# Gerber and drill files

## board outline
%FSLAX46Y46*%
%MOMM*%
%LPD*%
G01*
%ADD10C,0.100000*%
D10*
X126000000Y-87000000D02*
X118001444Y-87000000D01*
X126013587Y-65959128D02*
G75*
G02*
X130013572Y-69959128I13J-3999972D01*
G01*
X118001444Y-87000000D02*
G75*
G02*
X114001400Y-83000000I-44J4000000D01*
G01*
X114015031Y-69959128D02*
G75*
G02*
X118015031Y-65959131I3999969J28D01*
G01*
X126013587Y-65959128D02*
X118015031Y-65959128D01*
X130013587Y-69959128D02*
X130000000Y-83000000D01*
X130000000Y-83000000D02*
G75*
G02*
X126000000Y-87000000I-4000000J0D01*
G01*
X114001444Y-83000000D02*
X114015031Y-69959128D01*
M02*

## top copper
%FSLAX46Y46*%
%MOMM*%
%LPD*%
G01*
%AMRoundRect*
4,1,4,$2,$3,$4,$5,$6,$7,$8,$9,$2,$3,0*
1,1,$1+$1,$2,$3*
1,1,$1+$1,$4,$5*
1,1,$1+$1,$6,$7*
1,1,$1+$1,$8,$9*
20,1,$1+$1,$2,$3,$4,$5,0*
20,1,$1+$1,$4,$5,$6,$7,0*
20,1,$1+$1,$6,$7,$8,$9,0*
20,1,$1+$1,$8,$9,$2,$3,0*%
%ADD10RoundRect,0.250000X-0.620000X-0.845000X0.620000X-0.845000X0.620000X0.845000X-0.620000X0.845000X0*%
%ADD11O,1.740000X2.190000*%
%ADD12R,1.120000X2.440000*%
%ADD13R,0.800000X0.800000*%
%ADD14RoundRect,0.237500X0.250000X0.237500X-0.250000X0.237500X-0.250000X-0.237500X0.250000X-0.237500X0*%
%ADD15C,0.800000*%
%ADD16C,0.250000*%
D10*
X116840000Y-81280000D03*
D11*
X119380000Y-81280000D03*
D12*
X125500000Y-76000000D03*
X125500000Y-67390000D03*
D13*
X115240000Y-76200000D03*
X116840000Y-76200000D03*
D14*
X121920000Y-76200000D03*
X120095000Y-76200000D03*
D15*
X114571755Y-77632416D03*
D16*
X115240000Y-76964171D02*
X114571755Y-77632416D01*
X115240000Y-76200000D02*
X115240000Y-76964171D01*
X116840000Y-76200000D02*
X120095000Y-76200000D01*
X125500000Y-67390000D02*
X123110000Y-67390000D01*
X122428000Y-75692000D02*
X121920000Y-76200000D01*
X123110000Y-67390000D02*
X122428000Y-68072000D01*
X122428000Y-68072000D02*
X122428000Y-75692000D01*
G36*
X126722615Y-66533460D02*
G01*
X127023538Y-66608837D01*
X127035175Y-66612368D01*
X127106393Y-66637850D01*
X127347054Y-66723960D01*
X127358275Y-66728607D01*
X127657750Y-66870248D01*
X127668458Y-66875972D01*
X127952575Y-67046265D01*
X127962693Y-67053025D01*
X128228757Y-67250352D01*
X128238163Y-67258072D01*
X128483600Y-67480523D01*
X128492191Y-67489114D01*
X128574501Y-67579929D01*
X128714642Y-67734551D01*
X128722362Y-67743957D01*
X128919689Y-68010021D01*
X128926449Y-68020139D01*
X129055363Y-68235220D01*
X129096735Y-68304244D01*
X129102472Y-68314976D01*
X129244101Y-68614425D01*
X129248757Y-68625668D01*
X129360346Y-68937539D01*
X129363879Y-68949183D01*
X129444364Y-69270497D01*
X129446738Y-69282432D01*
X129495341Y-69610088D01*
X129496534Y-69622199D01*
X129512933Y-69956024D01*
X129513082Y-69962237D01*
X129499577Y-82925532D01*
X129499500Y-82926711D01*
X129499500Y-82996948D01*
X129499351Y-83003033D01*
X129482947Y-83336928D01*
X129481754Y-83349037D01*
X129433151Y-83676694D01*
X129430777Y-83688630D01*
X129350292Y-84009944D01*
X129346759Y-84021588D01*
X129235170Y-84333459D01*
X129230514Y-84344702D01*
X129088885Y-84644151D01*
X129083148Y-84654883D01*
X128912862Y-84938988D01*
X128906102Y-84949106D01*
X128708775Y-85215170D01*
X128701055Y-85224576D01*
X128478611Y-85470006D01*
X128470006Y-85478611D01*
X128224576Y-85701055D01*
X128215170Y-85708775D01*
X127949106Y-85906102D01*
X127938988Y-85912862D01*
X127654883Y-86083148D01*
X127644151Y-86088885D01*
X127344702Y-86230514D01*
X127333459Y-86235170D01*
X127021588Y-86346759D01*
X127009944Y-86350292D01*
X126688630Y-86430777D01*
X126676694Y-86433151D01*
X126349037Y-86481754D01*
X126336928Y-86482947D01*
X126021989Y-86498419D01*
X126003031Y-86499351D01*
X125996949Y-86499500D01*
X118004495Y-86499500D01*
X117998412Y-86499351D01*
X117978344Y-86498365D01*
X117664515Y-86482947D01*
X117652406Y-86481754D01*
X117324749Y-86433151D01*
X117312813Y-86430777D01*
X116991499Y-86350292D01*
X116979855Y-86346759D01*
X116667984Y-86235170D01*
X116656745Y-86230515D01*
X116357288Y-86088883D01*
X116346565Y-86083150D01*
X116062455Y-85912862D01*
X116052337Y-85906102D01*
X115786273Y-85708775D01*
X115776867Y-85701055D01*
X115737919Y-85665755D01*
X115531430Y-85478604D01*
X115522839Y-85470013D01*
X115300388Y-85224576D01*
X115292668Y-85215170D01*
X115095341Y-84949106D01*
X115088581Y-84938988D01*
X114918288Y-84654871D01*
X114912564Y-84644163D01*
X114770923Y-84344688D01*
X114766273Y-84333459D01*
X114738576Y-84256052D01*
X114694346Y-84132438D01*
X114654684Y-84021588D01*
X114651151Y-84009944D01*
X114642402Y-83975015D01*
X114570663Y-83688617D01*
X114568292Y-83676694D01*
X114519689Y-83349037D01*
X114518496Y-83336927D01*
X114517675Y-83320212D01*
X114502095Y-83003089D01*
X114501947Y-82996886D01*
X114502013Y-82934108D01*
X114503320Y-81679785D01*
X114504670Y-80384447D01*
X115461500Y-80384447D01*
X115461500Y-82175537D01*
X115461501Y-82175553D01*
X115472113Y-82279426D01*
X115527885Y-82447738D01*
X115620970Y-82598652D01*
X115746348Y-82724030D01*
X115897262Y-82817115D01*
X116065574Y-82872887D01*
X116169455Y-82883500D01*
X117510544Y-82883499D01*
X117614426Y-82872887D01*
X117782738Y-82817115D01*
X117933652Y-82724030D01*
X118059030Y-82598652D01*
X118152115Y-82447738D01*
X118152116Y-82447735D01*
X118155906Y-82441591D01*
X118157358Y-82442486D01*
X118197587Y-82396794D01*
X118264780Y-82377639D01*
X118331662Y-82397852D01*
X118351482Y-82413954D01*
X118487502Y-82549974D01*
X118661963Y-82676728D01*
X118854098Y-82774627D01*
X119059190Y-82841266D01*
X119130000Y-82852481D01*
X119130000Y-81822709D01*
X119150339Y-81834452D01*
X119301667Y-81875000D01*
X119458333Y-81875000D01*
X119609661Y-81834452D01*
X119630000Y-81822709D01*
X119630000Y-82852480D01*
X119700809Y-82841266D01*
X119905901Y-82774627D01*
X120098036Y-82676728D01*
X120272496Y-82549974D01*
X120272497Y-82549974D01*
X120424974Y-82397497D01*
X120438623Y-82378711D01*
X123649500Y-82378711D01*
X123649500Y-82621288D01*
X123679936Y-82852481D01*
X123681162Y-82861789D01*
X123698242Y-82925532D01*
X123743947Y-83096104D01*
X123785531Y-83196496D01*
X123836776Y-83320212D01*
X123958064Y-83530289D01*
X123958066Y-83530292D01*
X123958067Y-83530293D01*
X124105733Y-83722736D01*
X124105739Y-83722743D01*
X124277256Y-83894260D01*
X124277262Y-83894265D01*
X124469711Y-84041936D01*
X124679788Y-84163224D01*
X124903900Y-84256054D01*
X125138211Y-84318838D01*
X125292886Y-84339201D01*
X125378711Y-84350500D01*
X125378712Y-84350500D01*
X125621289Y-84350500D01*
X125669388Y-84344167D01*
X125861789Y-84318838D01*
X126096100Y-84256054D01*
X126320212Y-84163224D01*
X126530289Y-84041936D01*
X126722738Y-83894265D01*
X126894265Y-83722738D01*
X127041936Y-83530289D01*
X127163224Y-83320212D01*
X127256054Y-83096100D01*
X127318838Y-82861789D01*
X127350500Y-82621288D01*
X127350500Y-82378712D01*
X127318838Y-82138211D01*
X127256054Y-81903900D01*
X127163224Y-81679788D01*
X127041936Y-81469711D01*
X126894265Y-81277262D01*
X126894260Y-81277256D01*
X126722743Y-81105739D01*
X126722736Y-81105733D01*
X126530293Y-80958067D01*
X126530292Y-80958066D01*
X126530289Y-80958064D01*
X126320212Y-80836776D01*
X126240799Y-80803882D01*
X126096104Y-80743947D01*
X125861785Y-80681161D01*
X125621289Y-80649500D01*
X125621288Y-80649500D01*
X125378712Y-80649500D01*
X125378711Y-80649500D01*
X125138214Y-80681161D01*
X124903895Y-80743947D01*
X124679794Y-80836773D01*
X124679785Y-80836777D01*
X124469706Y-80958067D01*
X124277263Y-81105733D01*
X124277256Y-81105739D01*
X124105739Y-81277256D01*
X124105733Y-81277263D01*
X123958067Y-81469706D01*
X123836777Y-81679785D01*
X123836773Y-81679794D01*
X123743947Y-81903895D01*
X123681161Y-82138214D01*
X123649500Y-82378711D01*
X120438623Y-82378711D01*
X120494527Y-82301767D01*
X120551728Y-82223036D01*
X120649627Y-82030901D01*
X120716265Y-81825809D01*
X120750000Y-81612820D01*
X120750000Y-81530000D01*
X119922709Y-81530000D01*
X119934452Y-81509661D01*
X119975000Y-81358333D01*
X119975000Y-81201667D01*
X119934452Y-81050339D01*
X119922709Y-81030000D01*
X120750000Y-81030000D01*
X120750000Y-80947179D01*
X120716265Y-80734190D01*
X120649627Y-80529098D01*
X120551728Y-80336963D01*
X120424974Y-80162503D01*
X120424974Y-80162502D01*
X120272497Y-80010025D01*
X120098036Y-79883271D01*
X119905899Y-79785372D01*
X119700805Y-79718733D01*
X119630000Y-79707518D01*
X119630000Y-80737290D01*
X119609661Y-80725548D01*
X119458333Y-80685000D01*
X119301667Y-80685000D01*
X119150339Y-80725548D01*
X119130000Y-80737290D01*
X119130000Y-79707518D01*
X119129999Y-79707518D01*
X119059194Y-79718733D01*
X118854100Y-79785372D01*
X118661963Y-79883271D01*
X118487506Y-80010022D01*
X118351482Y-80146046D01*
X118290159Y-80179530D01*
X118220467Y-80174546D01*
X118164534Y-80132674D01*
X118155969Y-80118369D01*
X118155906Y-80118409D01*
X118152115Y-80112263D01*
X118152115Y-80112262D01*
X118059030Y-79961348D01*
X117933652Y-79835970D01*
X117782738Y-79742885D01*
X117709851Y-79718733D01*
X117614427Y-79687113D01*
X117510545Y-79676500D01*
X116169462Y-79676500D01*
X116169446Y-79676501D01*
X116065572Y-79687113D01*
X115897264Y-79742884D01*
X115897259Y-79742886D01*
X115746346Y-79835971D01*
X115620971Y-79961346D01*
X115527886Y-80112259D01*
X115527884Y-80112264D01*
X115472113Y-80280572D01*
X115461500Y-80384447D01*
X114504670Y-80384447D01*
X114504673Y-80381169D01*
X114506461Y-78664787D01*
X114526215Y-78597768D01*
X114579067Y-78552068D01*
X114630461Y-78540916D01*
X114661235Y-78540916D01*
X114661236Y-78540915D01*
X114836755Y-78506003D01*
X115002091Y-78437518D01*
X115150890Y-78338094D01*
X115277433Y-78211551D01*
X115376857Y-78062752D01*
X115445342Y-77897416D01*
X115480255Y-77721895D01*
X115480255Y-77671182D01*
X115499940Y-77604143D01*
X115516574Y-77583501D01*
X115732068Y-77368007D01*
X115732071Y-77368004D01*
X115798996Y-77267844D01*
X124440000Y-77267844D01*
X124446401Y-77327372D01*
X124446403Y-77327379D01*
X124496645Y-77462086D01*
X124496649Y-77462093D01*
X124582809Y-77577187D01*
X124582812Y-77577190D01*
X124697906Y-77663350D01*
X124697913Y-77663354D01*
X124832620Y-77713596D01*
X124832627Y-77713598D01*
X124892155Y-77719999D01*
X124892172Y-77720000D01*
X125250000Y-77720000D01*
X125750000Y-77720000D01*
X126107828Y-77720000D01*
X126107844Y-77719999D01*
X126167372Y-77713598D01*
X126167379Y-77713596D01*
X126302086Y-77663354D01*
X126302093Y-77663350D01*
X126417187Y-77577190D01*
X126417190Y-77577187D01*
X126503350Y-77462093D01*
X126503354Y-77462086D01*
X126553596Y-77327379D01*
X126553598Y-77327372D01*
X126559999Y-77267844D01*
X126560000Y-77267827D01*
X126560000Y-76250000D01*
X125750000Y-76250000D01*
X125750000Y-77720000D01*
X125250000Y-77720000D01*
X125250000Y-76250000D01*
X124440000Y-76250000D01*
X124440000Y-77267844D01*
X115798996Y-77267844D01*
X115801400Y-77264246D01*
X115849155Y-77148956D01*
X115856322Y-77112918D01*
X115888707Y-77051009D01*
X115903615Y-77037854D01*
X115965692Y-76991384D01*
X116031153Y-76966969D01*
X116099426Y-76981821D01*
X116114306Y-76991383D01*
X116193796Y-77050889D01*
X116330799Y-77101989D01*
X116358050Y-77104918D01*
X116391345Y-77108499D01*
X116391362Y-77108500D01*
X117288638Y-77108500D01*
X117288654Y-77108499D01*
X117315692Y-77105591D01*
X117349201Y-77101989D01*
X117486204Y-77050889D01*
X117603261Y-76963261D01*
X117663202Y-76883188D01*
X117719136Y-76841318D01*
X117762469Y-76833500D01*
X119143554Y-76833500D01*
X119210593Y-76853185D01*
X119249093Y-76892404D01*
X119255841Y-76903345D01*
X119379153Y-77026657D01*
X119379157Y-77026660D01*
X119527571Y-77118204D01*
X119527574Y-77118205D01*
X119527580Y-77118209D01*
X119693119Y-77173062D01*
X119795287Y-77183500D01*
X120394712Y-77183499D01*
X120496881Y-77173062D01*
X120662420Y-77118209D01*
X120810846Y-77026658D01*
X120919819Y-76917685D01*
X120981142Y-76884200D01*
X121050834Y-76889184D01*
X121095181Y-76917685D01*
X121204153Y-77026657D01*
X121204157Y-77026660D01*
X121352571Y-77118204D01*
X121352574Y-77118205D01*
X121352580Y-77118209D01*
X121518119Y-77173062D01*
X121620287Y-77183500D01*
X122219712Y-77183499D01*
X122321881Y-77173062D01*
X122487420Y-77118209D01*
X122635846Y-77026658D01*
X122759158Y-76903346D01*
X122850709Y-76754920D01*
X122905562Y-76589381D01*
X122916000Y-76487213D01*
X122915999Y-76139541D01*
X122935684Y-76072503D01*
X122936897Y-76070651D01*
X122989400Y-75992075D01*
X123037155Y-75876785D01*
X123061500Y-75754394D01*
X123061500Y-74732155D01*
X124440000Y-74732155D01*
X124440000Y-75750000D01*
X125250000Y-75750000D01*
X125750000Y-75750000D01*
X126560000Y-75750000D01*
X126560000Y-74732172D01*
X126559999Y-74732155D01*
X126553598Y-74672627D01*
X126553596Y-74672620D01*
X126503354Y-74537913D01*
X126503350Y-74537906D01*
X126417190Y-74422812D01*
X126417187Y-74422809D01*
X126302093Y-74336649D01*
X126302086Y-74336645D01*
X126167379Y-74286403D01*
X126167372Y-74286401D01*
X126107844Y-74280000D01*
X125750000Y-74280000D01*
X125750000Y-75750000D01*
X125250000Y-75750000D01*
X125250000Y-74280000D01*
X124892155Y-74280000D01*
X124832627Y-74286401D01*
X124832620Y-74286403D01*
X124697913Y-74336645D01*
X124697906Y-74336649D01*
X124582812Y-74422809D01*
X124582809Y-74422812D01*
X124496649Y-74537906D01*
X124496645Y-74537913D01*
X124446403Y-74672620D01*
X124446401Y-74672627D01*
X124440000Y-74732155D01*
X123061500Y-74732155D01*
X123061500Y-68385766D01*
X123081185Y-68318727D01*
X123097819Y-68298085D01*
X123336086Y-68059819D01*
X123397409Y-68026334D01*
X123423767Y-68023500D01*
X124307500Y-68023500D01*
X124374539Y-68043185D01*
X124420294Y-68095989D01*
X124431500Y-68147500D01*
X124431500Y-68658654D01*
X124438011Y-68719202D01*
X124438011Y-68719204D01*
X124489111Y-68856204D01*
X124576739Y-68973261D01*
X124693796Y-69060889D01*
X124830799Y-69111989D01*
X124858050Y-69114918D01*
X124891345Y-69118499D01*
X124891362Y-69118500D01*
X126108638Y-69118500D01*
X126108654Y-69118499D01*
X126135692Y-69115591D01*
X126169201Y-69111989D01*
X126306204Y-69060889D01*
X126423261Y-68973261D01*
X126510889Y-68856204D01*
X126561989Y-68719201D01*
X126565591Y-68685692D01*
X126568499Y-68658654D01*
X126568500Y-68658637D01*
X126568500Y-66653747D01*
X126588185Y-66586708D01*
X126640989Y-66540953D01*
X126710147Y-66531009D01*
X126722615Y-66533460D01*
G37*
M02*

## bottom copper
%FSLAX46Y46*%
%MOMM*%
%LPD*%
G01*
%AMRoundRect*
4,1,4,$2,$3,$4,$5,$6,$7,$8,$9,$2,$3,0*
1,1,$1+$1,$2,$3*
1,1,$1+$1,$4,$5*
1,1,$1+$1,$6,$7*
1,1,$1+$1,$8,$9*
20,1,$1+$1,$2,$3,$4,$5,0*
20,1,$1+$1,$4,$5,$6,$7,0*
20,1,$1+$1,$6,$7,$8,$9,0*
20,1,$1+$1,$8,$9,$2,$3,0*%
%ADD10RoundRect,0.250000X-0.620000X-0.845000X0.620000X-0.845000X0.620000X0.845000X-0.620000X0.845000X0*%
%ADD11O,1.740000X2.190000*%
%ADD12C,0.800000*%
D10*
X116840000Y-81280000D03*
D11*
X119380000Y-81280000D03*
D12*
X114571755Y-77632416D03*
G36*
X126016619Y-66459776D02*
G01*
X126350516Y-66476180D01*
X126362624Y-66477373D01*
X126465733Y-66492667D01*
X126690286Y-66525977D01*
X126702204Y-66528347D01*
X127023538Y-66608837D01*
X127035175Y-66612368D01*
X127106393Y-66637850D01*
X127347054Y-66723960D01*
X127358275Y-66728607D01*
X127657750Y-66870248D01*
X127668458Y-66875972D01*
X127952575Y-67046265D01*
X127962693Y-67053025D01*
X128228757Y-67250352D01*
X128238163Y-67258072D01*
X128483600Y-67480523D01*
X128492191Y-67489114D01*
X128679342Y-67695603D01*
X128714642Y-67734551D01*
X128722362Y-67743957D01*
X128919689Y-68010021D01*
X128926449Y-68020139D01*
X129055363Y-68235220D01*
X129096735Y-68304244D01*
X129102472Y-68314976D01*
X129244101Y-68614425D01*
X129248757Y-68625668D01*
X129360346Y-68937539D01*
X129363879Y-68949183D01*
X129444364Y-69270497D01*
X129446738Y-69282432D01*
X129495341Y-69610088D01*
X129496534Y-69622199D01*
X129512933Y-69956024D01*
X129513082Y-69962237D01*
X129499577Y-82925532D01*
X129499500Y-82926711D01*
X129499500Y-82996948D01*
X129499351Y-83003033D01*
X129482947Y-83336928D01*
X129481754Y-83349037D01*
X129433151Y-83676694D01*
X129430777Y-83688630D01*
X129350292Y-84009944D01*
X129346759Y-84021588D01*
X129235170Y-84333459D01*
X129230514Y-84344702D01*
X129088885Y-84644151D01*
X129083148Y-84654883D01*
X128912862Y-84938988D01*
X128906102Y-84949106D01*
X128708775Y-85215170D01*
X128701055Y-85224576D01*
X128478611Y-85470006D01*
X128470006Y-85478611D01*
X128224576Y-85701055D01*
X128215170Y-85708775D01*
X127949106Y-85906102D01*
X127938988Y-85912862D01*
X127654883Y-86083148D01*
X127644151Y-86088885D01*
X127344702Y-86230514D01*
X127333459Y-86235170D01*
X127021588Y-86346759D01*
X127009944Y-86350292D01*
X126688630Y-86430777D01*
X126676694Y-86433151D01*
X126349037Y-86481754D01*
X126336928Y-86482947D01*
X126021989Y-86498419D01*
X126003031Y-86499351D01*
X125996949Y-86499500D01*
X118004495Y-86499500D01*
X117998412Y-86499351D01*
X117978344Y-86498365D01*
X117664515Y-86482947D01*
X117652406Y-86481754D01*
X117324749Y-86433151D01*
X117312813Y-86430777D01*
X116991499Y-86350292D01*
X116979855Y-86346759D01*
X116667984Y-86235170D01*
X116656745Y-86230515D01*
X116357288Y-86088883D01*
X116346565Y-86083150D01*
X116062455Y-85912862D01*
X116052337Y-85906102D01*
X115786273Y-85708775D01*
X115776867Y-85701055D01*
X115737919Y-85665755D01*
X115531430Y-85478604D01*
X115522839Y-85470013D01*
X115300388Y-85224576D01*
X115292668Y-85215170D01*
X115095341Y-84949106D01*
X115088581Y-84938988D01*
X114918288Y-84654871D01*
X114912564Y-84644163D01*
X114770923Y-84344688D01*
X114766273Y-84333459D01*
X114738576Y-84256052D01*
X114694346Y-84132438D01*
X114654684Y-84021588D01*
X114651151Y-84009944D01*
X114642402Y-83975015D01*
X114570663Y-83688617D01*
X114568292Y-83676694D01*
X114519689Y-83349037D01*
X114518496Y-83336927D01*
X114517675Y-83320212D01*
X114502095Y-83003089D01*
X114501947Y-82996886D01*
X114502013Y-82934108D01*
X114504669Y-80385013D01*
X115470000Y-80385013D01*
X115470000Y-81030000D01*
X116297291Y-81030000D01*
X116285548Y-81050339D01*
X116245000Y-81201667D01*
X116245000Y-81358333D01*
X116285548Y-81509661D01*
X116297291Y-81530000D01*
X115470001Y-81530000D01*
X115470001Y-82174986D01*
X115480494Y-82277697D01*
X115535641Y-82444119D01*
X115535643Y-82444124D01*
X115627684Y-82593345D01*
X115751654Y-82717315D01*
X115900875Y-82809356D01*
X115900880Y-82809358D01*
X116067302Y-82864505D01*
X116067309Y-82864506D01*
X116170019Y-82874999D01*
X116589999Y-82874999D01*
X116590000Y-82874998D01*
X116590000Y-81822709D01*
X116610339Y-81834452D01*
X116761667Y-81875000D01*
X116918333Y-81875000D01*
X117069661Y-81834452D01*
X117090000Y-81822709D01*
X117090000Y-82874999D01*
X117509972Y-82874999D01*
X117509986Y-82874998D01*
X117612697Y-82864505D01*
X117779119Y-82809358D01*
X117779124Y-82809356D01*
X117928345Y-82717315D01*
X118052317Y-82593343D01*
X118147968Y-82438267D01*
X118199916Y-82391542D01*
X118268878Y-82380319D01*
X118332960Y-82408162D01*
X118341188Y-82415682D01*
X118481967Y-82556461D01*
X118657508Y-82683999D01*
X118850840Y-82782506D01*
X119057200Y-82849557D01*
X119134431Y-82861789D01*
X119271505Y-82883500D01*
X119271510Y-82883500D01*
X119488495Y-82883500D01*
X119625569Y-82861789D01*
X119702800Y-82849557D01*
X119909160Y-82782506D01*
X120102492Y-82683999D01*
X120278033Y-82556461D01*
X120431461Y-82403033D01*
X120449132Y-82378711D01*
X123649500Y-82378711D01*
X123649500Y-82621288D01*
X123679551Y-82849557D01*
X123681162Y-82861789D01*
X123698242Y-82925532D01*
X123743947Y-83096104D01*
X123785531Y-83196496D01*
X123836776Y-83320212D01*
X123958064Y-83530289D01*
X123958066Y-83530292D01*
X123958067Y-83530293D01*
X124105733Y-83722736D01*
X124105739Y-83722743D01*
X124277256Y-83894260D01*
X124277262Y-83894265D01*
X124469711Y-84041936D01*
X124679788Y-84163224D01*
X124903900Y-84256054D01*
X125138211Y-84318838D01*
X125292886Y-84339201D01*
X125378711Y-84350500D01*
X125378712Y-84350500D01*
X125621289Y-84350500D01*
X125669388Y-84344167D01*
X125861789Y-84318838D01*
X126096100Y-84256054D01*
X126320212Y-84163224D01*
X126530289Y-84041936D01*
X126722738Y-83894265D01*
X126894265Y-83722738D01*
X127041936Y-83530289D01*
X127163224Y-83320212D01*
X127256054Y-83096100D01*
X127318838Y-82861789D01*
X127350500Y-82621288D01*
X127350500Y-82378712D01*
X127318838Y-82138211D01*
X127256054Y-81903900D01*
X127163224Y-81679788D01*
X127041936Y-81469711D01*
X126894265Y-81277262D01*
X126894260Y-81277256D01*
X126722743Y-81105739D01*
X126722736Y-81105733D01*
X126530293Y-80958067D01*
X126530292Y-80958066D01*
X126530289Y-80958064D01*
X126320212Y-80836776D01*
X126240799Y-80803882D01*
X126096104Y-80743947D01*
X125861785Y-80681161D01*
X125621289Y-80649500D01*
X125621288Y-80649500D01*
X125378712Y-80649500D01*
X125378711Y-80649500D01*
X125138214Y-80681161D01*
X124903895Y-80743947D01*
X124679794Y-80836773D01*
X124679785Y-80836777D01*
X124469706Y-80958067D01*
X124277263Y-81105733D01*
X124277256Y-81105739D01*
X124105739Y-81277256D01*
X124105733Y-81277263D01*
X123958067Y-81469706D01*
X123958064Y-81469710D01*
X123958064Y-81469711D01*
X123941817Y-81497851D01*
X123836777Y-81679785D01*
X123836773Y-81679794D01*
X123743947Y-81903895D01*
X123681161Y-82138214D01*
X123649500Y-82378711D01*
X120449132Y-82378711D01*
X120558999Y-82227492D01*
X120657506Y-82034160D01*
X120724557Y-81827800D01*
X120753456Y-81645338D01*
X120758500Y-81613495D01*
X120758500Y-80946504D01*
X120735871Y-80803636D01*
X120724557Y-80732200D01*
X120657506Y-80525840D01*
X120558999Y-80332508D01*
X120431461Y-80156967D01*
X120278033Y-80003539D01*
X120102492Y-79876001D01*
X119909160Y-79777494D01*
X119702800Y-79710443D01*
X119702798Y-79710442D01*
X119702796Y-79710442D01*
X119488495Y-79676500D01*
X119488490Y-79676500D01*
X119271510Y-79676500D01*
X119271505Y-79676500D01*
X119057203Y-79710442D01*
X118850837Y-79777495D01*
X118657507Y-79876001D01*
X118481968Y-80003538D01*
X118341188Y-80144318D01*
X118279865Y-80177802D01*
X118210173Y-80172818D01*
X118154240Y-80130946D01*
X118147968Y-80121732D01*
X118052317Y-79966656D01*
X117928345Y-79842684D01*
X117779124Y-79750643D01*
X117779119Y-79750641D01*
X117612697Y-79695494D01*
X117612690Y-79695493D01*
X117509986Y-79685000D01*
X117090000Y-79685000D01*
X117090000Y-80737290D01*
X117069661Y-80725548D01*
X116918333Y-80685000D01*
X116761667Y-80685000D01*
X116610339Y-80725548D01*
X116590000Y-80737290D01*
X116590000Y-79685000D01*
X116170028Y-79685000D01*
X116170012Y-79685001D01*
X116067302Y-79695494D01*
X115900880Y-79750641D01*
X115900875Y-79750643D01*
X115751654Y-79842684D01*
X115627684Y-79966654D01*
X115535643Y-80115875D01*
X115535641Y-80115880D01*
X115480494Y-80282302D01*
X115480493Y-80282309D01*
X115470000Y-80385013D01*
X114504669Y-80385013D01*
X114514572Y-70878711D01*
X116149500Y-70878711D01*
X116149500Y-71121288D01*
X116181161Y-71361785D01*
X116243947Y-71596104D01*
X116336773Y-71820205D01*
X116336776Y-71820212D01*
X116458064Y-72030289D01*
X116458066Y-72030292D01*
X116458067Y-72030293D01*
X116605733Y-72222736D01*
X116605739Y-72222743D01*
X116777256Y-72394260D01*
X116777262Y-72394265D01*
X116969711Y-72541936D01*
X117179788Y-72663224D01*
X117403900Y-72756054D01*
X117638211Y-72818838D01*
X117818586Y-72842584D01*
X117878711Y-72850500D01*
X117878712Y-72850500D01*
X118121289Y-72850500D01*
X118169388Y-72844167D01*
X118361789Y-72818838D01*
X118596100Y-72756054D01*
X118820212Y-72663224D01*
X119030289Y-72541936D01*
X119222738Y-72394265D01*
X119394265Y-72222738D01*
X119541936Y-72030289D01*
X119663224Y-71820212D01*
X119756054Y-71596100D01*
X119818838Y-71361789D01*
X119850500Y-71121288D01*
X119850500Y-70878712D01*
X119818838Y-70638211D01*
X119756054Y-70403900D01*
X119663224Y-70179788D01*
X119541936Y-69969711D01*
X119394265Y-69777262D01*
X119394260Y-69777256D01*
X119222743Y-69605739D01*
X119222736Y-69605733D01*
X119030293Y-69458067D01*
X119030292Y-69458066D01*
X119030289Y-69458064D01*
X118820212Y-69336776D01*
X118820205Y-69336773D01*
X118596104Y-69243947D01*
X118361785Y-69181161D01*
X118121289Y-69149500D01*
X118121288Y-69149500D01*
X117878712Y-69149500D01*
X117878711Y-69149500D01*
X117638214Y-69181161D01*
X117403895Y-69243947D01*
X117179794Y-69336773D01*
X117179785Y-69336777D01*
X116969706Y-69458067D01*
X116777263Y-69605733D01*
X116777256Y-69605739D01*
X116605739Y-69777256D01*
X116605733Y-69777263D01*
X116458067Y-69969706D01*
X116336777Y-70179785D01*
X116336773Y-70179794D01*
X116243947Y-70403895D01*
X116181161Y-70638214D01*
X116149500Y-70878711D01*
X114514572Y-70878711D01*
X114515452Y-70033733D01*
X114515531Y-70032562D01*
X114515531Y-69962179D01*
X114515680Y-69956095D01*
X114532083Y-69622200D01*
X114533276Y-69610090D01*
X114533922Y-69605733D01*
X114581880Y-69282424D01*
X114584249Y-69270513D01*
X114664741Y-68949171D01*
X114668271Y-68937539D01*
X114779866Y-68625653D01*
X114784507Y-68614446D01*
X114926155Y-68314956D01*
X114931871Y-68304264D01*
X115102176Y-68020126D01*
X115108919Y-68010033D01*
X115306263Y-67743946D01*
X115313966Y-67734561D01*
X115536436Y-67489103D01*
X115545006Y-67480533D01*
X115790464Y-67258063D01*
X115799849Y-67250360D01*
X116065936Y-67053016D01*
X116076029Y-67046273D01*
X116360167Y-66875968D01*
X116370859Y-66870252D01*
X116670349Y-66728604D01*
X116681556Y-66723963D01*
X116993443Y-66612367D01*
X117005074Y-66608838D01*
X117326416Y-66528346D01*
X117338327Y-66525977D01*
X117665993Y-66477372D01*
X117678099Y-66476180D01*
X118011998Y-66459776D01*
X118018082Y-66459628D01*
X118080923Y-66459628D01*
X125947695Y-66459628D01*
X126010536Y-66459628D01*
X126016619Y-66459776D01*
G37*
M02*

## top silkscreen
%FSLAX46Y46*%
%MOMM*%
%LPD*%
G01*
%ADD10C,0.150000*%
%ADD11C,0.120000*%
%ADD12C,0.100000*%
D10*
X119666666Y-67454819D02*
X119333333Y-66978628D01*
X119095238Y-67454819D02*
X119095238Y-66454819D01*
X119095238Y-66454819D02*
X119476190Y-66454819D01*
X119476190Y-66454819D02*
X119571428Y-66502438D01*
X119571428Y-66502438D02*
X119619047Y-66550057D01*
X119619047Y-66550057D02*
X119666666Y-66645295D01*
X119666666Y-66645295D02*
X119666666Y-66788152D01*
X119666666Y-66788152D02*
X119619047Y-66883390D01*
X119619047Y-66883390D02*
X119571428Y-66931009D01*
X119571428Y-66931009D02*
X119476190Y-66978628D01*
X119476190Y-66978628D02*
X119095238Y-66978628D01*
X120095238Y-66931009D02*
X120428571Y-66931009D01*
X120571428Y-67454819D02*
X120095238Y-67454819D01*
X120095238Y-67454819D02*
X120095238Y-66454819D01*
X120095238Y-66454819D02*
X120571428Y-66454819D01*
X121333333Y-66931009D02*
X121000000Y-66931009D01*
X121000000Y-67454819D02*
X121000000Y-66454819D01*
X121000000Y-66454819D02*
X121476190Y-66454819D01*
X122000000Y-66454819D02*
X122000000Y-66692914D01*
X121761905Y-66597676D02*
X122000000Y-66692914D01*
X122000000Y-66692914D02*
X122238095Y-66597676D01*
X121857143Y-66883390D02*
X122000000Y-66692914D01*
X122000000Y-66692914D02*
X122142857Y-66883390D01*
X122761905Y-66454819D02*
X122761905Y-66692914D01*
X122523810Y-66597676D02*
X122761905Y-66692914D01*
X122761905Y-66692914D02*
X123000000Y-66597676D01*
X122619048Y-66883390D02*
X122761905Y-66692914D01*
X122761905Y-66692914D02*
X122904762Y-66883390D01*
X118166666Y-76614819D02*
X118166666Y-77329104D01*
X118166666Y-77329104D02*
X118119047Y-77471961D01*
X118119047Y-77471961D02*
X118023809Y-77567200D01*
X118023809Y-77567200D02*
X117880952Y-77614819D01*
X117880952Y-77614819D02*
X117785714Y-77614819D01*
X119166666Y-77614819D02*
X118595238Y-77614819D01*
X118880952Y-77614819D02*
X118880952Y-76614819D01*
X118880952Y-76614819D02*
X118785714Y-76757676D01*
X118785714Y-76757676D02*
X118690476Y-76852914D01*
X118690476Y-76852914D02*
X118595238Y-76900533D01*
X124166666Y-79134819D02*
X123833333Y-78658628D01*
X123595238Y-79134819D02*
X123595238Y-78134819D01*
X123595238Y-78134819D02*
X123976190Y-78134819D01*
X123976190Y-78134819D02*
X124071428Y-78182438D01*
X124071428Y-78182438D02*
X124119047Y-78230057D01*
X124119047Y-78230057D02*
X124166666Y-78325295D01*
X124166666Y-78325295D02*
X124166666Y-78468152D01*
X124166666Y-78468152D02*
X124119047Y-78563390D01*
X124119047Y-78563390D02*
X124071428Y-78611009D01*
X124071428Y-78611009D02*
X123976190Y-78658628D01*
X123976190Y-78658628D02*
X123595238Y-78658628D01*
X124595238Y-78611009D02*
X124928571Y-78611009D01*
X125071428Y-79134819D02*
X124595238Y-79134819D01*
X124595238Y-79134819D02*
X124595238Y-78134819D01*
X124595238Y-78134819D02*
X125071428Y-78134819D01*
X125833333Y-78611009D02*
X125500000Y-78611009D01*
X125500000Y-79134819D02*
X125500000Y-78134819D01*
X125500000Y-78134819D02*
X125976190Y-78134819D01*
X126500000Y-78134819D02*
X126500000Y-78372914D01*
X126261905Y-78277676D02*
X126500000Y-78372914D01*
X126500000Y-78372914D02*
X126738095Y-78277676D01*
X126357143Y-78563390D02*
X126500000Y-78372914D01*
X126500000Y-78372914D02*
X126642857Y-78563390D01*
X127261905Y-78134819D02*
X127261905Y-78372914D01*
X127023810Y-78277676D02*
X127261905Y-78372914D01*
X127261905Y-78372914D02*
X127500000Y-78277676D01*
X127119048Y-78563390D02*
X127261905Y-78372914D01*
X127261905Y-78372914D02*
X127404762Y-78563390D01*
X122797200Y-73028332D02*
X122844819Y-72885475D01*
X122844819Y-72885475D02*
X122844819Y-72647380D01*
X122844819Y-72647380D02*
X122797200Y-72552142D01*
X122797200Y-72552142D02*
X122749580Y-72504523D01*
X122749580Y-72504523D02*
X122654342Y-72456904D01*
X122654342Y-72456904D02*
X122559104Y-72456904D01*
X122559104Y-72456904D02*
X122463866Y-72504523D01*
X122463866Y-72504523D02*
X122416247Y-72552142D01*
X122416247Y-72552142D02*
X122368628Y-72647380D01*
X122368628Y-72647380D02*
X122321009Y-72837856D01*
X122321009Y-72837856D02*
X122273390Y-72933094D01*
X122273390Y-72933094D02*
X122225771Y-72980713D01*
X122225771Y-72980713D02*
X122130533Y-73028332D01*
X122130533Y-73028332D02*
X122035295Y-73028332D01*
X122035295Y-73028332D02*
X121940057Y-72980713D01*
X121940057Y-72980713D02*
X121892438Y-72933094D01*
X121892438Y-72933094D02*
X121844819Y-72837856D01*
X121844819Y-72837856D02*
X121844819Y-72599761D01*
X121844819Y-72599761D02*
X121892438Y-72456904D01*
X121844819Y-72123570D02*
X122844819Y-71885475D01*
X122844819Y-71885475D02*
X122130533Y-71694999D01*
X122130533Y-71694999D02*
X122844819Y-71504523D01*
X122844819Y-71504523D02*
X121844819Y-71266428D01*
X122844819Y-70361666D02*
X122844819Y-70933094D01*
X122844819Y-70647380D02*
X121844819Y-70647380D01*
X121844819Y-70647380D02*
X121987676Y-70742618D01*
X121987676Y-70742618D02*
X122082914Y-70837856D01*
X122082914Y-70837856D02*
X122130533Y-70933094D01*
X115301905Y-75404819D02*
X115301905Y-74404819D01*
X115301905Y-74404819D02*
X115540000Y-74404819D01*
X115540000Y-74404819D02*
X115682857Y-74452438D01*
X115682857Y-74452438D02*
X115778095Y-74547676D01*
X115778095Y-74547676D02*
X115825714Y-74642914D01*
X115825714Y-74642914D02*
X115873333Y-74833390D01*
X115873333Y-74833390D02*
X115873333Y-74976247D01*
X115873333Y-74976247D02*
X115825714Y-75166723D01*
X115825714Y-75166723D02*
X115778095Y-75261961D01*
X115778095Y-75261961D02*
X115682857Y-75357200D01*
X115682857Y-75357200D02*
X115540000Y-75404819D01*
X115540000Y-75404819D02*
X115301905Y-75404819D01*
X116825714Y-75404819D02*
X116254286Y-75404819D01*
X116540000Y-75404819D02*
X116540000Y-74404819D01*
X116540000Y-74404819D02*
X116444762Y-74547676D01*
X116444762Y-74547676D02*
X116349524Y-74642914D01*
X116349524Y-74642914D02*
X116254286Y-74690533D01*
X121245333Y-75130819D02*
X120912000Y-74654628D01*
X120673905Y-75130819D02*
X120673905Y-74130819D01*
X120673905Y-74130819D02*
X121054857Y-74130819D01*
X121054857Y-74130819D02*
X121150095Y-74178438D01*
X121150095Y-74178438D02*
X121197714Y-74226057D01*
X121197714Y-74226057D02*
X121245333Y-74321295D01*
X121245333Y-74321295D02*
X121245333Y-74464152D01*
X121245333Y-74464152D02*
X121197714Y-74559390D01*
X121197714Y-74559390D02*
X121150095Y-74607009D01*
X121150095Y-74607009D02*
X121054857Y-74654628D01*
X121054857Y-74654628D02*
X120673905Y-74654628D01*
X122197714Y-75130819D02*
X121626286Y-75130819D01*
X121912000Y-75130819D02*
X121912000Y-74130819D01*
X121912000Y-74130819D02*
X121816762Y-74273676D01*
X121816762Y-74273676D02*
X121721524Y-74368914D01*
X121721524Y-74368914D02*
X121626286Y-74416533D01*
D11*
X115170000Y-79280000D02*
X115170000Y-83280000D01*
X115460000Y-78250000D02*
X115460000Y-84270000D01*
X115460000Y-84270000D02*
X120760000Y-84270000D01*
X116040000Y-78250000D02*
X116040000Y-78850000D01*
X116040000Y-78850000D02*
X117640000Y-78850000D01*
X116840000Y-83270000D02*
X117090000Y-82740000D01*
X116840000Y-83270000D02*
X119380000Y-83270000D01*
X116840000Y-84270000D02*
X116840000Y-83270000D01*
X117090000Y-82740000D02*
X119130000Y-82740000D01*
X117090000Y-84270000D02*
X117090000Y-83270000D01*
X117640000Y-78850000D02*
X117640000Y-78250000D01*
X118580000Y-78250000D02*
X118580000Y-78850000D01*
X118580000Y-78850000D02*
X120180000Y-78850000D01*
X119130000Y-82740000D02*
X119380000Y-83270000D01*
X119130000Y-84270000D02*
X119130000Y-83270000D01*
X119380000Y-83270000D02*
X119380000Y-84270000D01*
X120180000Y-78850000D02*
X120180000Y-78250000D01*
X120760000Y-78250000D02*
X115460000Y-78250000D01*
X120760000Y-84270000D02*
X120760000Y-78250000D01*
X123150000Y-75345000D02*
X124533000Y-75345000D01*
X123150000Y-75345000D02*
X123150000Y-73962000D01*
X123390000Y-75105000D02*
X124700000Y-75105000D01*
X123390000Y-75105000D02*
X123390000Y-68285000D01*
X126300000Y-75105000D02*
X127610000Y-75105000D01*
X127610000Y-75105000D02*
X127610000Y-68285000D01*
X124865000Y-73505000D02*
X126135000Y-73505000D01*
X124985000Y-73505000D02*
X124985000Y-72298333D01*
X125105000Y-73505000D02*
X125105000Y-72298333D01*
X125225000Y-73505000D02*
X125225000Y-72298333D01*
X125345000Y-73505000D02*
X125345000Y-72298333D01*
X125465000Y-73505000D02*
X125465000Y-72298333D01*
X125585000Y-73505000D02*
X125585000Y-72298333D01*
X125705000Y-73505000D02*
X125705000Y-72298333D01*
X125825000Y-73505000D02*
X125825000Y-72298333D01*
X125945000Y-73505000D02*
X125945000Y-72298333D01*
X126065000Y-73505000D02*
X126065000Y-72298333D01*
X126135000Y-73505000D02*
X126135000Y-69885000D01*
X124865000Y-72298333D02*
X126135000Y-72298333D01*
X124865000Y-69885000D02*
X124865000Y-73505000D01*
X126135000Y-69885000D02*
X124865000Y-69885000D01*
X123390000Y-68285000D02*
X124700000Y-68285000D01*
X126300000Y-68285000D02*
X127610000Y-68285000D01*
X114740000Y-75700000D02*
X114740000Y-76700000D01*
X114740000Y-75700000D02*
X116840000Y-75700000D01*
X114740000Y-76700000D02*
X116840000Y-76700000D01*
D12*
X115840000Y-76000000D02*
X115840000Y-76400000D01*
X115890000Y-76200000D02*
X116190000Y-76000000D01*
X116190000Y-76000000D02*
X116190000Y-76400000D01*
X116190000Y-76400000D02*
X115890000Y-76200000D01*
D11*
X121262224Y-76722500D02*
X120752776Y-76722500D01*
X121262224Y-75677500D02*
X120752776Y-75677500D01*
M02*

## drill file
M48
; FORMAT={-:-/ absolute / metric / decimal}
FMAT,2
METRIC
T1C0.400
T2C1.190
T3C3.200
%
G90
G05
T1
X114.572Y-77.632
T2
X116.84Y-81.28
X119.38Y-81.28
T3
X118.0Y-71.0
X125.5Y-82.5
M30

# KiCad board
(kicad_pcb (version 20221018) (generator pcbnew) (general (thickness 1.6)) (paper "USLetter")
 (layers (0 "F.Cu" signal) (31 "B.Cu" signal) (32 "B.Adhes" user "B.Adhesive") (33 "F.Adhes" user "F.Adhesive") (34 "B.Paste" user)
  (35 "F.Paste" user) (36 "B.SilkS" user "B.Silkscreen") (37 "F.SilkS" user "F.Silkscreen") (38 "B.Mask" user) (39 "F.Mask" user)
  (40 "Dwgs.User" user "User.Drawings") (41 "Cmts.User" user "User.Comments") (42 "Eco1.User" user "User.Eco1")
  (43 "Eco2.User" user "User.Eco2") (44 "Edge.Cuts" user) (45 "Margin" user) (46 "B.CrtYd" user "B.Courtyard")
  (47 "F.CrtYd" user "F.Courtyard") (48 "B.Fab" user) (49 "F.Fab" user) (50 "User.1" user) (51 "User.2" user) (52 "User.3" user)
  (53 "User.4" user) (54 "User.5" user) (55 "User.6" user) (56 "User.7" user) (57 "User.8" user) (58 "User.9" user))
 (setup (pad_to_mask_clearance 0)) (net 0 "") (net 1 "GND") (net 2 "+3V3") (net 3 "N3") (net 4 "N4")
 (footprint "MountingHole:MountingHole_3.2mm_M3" (layer "F.Cu") (at 118 71)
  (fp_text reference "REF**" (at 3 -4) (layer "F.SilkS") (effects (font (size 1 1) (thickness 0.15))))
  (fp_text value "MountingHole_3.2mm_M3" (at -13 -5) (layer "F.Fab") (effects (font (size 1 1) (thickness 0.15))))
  (pad "" np_thru_hole circle (at 0 0) (size 3.2 3.2) (drill 3.2) (layers "*.Cu" "*.Mask")))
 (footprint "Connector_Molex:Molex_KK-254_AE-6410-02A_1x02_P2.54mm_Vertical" (layer "F.Cu") (at 116.84 81.28)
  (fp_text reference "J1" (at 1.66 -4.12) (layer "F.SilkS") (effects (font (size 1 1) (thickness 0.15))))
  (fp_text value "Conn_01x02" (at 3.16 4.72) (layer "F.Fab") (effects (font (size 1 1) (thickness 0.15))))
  (fp_line (start -1.67 -2) (end -1.67 2) (stroke (width 0.12) (type solid)) (layer "F.SilkS"))
  (fp_line (start -1.38 -3.03) (end -1.38 2.99) (stroke (width 0.12) (type solid)) (layer "F.SilkS"))
  (fp_line (start -1.38 2.99) (end 3.92 2.99) (stroke (width 0.12) (type solid)) (layer "F.SilkS"))
  (fp_line (start -0.8 -3.03) (end -0.8 -2.43) (stroke (width 0.12) (type solid)) (layer "F.SilkS"))
  (fp_line (start -0.8 -2.43) (end 0.8 -2.43) (stroke (width 0.12) (type solid)) (layer "F.SilkS"))
  (fp_line (start 0 1.99) (end 0.25 1.46) (stroke (width 0.12) (type solid)) (layer "F.SilkS"))
  (fp_line (start 0 1.99) (end 2.54 1.99) (stroke (width 0.12) (type solid)) (layer "F.SilkS"))
  (fp_line (start 0 2.99) (end 0 1.99) (stroke (width 0.12) (type solid)) (layer "F.SilkS"))
  (fp_line (start 0.25 1.46) (end 2.29 1.46) (stroke (width 0.12) (type solid)) (layer "F.SilkS"))
  (fp_line (start 0.25 2.99) (end 0.25 1.99) (stroke (width 0.12) (type solid)) (layer "F.SilkS"))
  (fp_line (start 0.8 -2.43) (end 0.8 -3.03) (stroke (width 0.12) (type solid)) (layer "F.SilkS"))
  (fp_line (start 1.74 -3.03) (end 1.74 -2.43) (stroke (width 0.12) (type solid)) (layer "F.SilkS"))
  (fp_line (start 1.74 -2.43) (end 3.34 -2.43) (stroke (width 0.12) (type solid)) (layer "F.SilkS"))
  (fp_line (start 2.29 1.46) (end 2.54 1.99) (stroke (width 0.12) (type solid)) (layer "F.SilkS"))
  (fp_line (start 2.29 2.99) (end 2.29 1.99) (stroke (width 0.12) (type solid)) (layer "F.SilkS"))
  (fp_line (start 2.54 1.99) (end 2.54 2.99) (stroke (width 0.12) (type solid)) (layer "F.SilkS"))
  (fp_line (start 3.34 -2.43) (end 3.34 -3.03) (stroke (width 0.12) (type solid)) (layer "F.SilkS"))
  (fp_line (start 3.92 -3.03) (end -1.38 -3.03) (stroke (width 0.12) (type solid)) (layer "F.SilkS"))
  (fp_line (start 3.92 2.99) (end 3.92 -3.03) (stroke (width 0.12) (type solid)) (layer "F.SilkS"))
  (pad "1" thru_hole roundrect (at 0 0) (size 1.74 2.19) (drill 1.19) (layers "*.Cu" "*.Mask") (roundrect_rratio 0.143678) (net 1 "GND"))
  (pad "2" thru_hole oval (at 2.54 0) (size 1.74 2.19) (drill 1.19) (layers "*.Cu" "*.Mask") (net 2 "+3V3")))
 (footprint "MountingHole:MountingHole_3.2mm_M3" (layer "F.Cu") (at 125.5 82.5)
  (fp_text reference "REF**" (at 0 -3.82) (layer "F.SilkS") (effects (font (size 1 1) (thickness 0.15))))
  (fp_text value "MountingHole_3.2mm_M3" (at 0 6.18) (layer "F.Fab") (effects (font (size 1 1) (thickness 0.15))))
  (pad "" np_thru_hole circle (at 0 0) (size 3.2 3.2) (drill 3.2) (layers "F&B.Cu" "*.Mask")))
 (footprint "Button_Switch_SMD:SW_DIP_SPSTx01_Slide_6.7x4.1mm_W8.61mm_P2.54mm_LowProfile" (layer "F.Cu") (at 125.5 71.695 90)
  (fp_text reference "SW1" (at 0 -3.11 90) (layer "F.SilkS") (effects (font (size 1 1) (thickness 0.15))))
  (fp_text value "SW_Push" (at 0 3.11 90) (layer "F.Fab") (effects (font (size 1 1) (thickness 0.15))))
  (fp_line (start -3.65 -2.35) (end -3.65 -0.967) (stroke (width 0.12) (type solid)) (layer "F.SilkS"))
  (fp_line (start -3.65 -2.35) (end -2.267 -2.35) (stroke (width 0.12) (type solid)) (layer "F.SilkS"))
  (fp_line (start -3.41 -2.11) (end -3.41 -0.8) (stroke (width 0.12) (type solid)) (layer "F.SilkS"))
  (fp_line (start -3.41 -2.11) (end 3.41 -2.11) (stroke (width 0.12) (type solid)) (layer "F.SilkS"))
  (fp_line (start -3.41 0.8) (end -3.41 2.11) (stroke (width 0.12) (type solid)) (layer "F.SilkS"))
  (fp_line (start -3.41 2.11) (end 3.41 2.11) (stroke (width 0.12) (type solid)) (layer "F.SilkS"))
  (fp_line (start -1.81 -0.635) (end -1.81 0.635) (stroke (width 0.12) (type solid)) (layer "F.SilkS"))
  (fp_line (start -1.81 -0.515) (end -0.603333 -0.515) (stroke (width 0.12) (type solid)) (layer "F.SilkS"))
  (fp_line (start -1.81 -0.395) (end -0.603333 -0.395) (stroke (width 0.12) (type solid)) (layer "F.SilkS"))
  (fp_line (start -1.81 -0.275) (end -0.603333 -0.275) (stroke (width 0.12) (type solid)) (layer "F.SilkS"))
  (fp_line (start -1.81 -0.155) (end -0.603333 -0.155) (stroke (width 0.12) (type solid)) (layer "F.SilkS"))
  (fp_line (start -1.81 -0.035) (end -0.603333 -0.035) (stroke (width 0.12) (type solid)) (layer "F.SilkS"))
  (fp_line (start -1.81 0.085) (end -0.603333 0.085) (stroke (width 0.12) (type solid)) (layer "F.SilkS"))
  (fp_line (start -1.81 0.205) (end -0.603333 0.205) (stroke (width 0.12) (type solid)) (layer "F.SilkS"))
  (fp_line (start -1.81 0.325) (end -0.603333 0.325) (stroke (width 0.12) (type solid)) (layer "F.SilkS"))
  (fp_line (start -1.81 0.445) (end -0.603333 0.445) (stroke (width 0.12) (type solid)) (layer "F.SilkS"))
  (fp_line (start -1.81 0.565) (end -0.603333 0.565) (stroke (width 0.12) (type solid)) (layer "F.SilkS"))
  (fp_line (start -1.81 0.635) (end 1.81 0.635) (stroke (width 0.12) (type solid)) (layer "F.SilkS"))
  (fp_line (start -0.603333 -0.635) (end -0.603333 0.635) (stroke (width 0.12) (type solid)) (layer "F.SilkS"))
  (fp_line (start 1.81 -0.635) (end -1.81 -0.635) (stroke (width 0.12) (type solid)) (layer "F.SilkS"))
  (fp_line (start 1.81 0.635) (end 1.81 -0.635) (stroke (width 0.12) (type solid)) (layer "F.SilkS"))
  (fp_line (start 3.41 -2.11) (end 3.41 -0.8) (stroke (width 0.12) (type solid)) (layer "F.SilkS"))
  (fp_line (start 3.41 0.8) (end 3.41 2.11) (stroke (width 0.12) (type solid)) (layer "F.SilkS"))
  (pad "1" smd rect (at -4.305 0 90) (size 2.44 1.12) (layers "F.Cu" "F.Paste" "F.Mask") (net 2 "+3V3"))
  (pad "2" smd rect (at 4.305 0 90) (size 2.44 1.12) (layers "F.Cu" "F.Paste" "F.Mask") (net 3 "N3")))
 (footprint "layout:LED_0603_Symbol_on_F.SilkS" (layer "F.Cu") (at 116.04 76.2)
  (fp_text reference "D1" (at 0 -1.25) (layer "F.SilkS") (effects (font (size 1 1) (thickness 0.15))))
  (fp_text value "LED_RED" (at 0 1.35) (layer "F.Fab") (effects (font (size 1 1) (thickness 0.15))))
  (fp_line (start -1.3 -0.5) (end -1.3 0.5) (stroke (width 0.12) (type solid)) (layer "F.SilkS"))
  (fp_line (start -1.3 -0.5) (end 0.8 -0.5) (stroke (width 0.12) (type solid)) (layer "F.SilkS"))
  (fp_line (start -1.3 0.5) (end 0.8 0.5) (stroke (width 0.12) (type solid)) (layer "F.SilkS"))
  (fp_line (start -0.2 -0.2) (end -0.2 0.2) (stroke (width 0.1) (type solid)) (layer "F.SilkS"))
  (fp_line (start -0.15 0) (end 0.15 -0.2) (stroke (width 0.1) (type solid)) (layer "F.SilkS"))
  (fp_line (start 0.15 -0.2) (end 0.15 0.2) (stroke (width 0.1) (type solid)) (layer "F.SilkS"))
  (fp_line (start 0.15 0.2) (end -0.15 0) (stroke (width 0.1) (type solid)) (layer "F.SilkS"))
  (pad "1" smd rect (at -0.8 0 180) (size 0.8 0.8) (layers "F.Cu" "F.Paste" "F.Mask") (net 1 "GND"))
  (pad "2" smd rect (at 0.8 0 180) (size 0.8 0.8) (layers "F.Cu" "F.Paste" "F.Mask") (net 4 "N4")))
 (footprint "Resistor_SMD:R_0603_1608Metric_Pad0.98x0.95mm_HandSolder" (layer "F.Cu") (at 121.0075 76.2 180)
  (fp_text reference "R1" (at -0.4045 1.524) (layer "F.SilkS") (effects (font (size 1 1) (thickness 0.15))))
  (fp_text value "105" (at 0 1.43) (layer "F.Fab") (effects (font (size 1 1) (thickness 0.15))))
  (fp_line (start -0.254724 -0.5225) (end 0.254724 -0.5225) (stroke (width 0.12) (type solid)) (layer "F.SilkS"))
  (fp_line (start -0.254724 0.5225) (end 0.254724 0.5225) (stroke (width 0.12) (type solid)) (layer "F.SilkS"))
  (pad "1" smd roundrect (at -0.9125 0 180) (size 0.975 0.95) (layers "F.Cu" "F.Paste" "F.Mask") (roundrect_rratio 0.25) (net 3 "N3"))
  (pad "2" smd roundrect (at 0.9125 0 180) (size 0.975 0.95) (layers "F.Cu" "F.Paste" "F.Mask") (roundrect_rratio 0.25) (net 4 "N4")))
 (gr_line (start 126 87) (end 118.001444 87) (stroke (width 0.1) (type default)) (layer "Edge.Cuts"))
 (gr_arc (start 126.013587 65.959128) (mid 128.842014 67.130701) (end 130.013587 69.959128) (stroke (width 0.1) (type default))
  (layer "Edge.Cuts"))
 (gr_arc (start 118.001444 87) (mid 115.173017 85.828427) (end 114.001444 83) (stroke (width 0.1) (type default)) (layer "Edge.Cuts"))
 (gr_arc (start 114.015031 69.959128) (mid 115.186604 67.130701) (end 118.015031 65.959128) (stroke (width 0.1) (type default))
  (layer "Edge.Cuts"))
 (gr_line (start 126.013587 65.959128) (end 118.015031 65.959128) (stroke (width 0.1) (type default)) (layer "Edge.Cuts"))
 (gr_line (start 130.013587 69.959128) (end 130 83) (stroke (width 0.1) (type default)) (layer "Edge.Cuts"))
 (gr_arc (start 130 83) (mid 128.828427 85.828427) (end 126 87) (stroke (width 0.1) (type default)) (layer "Edge.Cuts"))
 (gr_line (start 114.001444 83) (end 114.015031 69.959128) (stroke (width 0.1) (type default)) (layer "Edge.Cuts"))
 (segment (start 115.24 76.964171) (end 114.571755 77.632416) (width 0.25) (layer "F.Cu") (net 1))
 (segment (start 115.24 76.2) (end 115.24 76.964171) (width 0.25) (layer "F.Cu") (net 1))
 (via (at 114.571755 77.632416) (size 0.8) (drill 0.4) (layers "F.Cu" "B.Cu") (free) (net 1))
 (segment (start 116.84 76.2) (end 120.095 76.2) (width 0.25) (layer "F.Cu") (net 4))
 (segment (start 125.5 67.39) (end 123.11 67.39) (width 0.25) (layer "F.Cu") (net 3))
 (segment (start 122.428 75.692) (end 121.92 76.2) (width 0.25) (layer "F.Cu") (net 3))
 (segment (start 123.11 67.39) (end 122.428 68.072) (width 0.25) (layer "F.Cu") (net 3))
 (segment (start 122.428 68.072) (end 122.428 75.692) (width 0.25) (layer "F.Cu") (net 3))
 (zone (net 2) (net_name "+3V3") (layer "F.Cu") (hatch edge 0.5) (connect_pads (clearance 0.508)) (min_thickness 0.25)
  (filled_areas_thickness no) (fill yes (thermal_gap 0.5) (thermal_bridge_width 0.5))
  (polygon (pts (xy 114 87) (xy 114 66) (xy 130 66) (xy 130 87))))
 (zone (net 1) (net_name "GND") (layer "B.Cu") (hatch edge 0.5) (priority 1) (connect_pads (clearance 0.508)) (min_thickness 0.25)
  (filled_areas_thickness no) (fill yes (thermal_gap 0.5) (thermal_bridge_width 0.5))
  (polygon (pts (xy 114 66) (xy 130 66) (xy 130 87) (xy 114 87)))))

